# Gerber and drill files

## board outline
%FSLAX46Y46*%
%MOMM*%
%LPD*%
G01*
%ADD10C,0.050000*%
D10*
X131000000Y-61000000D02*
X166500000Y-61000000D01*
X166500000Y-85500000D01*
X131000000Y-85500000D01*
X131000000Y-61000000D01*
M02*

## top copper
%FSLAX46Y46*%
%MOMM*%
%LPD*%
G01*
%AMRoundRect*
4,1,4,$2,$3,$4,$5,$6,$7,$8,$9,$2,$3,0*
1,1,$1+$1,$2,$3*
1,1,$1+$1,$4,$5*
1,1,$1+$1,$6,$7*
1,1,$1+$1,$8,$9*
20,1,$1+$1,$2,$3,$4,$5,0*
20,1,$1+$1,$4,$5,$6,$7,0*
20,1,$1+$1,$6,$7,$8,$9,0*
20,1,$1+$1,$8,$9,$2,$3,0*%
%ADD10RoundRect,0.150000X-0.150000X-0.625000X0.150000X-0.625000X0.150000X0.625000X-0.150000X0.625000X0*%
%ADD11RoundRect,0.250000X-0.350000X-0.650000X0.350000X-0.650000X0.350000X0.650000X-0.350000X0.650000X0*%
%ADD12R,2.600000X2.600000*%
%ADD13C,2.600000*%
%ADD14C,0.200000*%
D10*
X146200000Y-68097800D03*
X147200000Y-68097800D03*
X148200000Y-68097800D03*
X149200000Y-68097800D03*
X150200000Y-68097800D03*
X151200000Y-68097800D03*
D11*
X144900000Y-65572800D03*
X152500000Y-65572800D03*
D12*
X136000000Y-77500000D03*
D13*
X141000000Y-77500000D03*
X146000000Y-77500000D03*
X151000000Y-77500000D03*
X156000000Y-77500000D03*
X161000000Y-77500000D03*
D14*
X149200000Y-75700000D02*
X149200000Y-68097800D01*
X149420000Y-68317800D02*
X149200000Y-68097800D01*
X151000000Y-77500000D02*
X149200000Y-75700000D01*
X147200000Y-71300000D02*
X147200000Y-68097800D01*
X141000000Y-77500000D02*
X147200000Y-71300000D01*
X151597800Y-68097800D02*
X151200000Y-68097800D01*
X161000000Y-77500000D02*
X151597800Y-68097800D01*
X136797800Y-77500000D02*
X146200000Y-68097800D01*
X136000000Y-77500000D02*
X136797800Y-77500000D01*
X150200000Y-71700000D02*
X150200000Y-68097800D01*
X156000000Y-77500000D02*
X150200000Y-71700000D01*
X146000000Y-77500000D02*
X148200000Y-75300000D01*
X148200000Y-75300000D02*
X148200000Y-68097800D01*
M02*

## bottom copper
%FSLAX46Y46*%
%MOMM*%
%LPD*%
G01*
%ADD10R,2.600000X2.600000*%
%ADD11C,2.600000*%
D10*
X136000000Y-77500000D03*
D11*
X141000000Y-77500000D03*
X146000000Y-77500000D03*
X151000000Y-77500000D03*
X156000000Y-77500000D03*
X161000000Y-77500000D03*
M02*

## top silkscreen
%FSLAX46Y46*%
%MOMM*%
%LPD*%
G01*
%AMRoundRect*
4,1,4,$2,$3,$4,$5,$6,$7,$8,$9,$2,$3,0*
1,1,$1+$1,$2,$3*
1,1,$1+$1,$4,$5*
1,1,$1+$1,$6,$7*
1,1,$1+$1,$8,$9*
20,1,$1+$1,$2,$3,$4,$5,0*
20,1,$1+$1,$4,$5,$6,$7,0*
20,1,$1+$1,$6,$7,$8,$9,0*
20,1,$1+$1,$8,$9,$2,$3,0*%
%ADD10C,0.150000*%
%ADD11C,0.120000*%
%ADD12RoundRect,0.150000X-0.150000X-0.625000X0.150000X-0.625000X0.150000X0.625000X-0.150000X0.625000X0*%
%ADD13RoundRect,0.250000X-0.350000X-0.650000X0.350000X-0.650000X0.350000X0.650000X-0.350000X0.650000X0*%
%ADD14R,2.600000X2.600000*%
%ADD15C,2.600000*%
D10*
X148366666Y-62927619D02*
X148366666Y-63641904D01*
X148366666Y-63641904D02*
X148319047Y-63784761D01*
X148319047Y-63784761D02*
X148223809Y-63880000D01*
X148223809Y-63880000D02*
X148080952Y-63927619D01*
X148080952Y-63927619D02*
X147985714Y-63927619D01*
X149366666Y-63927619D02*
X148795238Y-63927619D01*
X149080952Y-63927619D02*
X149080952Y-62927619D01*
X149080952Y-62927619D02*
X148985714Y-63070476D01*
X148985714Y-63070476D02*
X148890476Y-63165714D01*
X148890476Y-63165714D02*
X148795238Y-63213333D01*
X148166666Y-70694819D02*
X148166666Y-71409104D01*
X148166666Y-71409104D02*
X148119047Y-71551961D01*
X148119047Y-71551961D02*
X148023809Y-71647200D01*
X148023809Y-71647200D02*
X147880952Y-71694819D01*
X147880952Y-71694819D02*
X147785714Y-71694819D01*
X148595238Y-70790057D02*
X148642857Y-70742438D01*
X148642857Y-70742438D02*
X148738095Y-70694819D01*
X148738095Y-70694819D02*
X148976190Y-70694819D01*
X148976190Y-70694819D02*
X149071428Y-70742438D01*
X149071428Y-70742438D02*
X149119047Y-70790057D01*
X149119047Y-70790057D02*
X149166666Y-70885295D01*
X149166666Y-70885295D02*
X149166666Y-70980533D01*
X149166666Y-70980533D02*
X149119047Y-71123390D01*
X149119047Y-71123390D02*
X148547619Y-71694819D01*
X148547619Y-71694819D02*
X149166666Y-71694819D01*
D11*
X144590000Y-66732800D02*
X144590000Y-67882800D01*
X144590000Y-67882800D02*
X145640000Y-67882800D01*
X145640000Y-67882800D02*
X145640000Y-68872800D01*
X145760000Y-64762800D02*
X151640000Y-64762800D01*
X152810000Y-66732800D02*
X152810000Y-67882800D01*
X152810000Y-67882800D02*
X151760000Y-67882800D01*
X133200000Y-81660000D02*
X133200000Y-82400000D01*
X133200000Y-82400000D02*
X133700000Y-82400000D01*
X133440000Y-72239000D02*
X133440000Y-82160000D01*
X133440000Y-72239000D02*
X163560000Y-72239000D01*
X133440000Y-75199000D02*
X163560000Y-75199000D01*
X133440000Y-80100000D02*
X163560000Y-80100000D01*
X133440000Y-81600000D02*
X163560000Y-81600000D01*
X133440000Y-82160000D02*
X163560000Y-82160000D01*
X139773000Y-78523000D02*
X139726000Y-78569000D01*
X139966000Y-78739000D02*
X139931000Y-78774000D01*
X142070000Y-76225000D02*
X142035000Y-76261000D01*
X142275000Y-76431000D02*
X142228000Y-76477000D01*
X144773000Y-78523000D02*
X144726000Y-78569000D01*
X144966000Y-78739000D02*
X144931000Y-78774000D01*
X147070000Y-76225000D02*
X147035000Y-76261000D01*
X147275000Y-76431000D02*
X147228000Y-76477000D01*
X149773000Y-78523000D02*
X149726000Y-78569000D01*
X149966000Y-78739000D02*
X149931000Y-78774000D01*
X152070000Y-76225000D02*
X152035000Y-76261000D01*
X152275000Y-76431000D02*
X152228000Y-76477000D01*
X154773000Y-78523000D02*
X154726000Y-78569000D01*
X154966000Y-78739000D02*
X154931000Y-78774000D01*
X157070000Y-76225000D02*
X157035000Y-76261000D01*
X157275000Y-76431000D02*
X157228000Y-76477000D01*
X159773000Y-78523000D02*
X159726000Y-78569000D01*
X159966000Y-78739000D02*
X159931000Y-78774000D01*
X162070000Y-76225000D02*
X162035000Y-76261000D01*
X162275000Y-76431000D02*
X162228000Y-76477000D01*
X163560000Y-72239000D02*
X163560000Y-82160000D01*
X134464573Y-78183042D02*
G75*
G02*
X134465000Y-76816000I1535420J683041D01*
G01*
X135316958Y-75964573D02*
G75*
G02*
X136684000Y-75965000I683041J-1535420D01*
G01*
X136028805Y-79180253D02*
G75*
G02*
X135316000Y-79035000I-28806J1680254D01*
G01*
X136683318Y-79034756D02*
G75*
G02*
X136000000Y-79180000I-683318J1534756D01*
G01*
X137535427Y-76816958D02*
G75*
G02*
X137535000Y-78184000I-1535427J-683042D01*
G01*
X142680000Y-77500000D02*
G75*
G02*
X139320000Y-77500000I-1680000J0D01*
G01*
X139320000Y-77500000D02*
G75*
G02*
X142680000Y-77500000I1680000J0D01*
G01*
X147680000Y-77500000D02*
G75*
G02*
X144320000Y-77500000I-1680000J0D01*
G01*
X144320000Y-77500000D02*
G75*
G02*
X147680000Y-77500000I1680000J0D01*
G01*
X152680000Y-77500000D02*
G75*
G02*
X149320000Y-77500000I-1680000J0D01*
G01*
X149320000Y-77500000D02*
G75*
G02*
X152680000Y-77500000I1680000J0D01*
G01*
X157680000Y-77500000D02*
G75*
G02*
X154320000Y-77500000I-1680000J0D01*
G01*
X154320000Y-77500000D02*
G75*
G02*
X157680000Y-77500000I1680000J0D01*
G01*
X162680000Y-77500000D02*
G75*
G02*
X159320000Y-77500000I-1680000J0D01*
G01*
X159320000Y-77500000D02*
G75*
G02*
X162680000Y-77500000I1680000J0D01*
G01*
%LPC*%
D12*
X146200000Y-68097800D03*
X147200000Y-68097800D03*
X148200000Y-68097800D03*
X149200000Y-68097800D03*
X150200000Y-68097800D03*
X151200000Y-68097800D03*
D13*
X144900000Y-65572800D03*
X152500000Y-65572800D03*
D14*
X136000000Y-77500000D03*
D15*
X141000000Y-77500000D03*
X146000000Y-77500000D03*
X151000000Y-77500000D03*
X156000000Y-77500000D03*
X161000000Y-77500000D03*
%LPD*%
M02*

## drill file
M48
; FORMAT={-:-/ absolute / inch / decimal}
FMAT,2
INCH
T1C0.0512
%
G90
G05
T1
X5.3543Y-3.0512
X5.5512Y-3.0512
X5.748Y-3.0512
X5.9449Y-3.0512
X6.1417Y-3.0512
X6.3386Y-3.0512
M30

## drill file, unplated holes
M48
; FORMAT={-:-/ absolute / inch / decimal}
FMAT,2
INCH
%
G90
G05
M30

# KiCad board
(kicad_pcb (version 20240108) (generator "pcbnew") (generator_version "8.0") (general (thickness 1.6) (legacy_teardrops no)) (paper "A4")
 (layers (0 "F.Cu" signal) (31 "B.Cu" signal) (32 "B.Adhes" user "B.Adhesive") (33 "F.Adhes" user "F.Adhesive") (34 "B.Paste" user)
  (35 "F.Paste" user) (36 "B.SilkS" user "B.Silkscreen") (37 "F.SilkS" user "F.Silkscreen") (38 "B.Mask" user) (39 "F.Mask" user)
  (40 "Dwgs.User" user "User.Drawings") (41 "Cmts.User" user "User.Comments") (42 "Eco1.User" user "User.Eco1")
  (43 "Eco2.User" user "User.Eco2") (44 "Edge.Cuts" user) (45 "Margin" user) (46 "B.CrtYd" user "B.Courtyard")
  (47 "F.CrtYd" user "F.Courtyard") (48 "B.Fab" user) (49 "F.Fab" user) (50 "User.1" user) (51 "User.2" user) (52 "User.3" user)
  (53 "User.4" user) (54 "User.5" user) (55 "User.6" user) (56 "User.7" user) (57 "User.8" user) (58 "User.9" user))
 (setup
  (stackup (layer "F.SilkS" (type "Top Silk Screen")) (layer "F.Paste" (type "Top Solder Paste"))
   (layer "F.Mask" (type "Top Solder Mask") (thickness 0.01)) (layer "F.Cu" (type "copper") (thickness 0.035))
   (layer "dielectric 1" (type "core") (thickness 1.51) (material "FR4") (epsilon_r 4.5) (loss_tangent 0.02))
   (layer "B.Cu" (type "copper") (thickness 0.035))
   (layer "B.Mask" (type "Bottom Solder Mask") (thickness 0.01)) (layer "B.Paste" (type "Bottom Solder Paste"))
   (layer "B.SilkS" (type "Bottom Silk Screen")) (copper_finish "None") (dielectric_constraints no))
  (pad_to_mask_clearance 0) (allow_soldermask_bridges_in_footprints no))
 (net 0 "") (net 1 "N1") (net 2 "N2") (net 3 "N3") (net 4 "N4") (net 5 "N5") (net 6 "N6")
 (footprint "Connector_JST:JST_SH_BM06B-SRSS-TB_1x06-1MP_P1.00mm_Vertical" (layer "F.Cu") (at 148.7 66.7728)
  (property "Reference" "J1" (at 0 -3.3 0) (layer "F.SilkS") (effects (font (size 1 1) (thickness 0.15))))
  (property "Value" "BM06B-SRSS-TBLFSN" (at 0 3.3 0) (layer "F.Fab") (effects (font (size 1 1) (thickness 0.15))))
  (fp_line (start -4.11 -0.04) (end -4.11 1.11) (stroke (width 0.12) (type solid)) (layer "F.SilkS"))
  (fp_line (start -4.11 1.11) (end -3.06 1.11) (stroke (width 0.12) (type solid)) (layer "F.SilkS"))
  (fp_line (start -3.06 1.11) (end -3.06 2.1) (stroke (width 0.12) (type solid)) (layer "F.SilkS"))
  (fp_line (start -2.94 -2.01) (end 2.94 -2.01) (stroke (width 0.12) (type solid)) (layer "F.SilkS"))
  (fp_line (start 4.11 -0.04) (end 4.11 1.11) (stroke (width 0.12) (type solid)) (layer "F.SilkS"))
  (fp_line (start 4.11 1.11) (end 3.06 1.11) (stroke (width 0.12) (type solid)) (layer "F.SilkS"))
  (pad "1" smd roundrect (at -2.5 1.325) (size 0.6 1.55) (layers "F.Cu" "F.Paste" "F.Mask") (roundrect_rratio 0.25) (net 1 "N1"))
  (pad "2" smd roundrect (at -1.5 1.325) (size 0.6 1.55) (layers "F.Cu" "F.Paste" "F.Mask") (roundrect_rratio 0.25) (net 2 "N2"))
  (pad "3" smd roundrect (at -0.5 1.325) (size 0.6 1.55) (layers "F.Cu" "F.Paste" "F.Mask") (roundrect_rratio 0.25) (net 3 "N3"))
  (pad "4" smd roundrect (at 0.5 1.325) (size 0.6 1.55) (layers "F.Cu" "F.Paste" "F.Mask") (roundrect_rratio 0.25) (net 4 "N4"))
  (pad "5" smd roundrect (at 1.5 1.325) (size 0.6 1.55) (layers "F.Cu" "F.Paste" "F.Mask") (roundrect_rratio 0.25) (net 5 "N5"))
  (pad "6" smd roundrect (at 2.5 1.325) (size 0.6 1.55) (layers "F.Cu" "F.Paste" "F.Mask") (roundrect_rratio 0.25) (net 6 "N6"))
  (pad "MP" smd roundrect (at -3.8 -1.2) (size 1.2 1.8) (layers "F.Cu" "F.Paste" "F.Mask") (roundrect_rratio 0.208333))
  (pad "MP" smd roundrect (at 3.8 -1.2) (size 1.2 1.8) (layers "F.Cu" "F.Paste" "F.Mask") (roundrect_rratio 0.208333)))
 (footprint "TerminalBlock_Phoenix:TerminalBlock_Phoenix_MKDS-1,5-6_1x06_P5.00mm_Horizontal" (layer "F.Cu") (at 136 77.5)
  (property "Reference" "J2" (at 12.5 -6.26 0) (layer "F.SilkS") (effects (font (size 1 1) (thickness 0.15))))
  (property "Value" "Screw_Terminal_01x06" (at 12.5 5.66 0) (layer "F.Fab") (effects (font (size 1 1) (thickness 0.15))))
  (fp_line (start -2.8 4.16) (end -2.8 4.9) (stroke (width 0.12) (type solid)) (layer "F.SilkS"))
  (fp_line (start -2.8 4.9) (end -2.3 4.9) (stroke (width 0.12) (type solid)) (layer "F.SilkS"))
  (fp_line (start -2.56 -5.261) (end -2.56 4.66) (stroke (width 0.12) (type solid)) (layer "F.SilkS"))
  (fp_line (start -2.56 -5.261) (end 27.56 -5.261) (stroke (width 0.12) (type solid)) (layer "F.SilkS"))
  (fp_line (start -2.56 -2.301) (end 27.56 -2.301) (stroke (width 0.12) (type solid)) (layer "F.SilkS"))
  (fp_line (start -2.56 2.6) (end 27.56 2.6) (stroke (width 0.12) (type solid)) (layer "F.SilkS"))
  (fp_line (start -2.56 4.1) (end 27.56 4.1) (stroke (width 0.12) (type solid)) (layer "F.SilkS"))
  (fp_line (start -2.56 4.66) (end 27.56 4.66) (stroke (width 0.12) (type solid)) (layer "F.SilkS"))
  (fp_line (start 3.773 1.023) (end 3.726 1.069) (stroke (width 0.12) (type solid)) (layer "F.SilkS"))
  (fp_line (start 3.966 1.239) (end 3.931 1.274) (stroke (width 0.12) (type solid)) (layer "F.SilkS"))
  (fp_line (start 6.07 -1.275) (end 6.035 -1.239) (stroke (width 0.12) (type solid)) (layer "F.SilkS"))
  (fp_line (start 6.275 -1.069) (end 6.228 -1.023) (stroke (width 0.12) (type solid)) (layer "F.SilkS"))
  (fp_line (start 8.773 1.023) (end 8.726 1.069) (stroke (width 0.12) (type solid)) (layer "F.SilkS"))
  (fp_line (start 8.966 1.239) (end 8.931 1.274) (stroke (width 0.12) (type solid)) (layer "F.SilkS"))
  (fp_line (start 11.07 -1.275) (end 11.035 -1.239) (stroke (width 0.12) (type solid)) (layer "F.SilkS"))
  (fp_line (start 11.275 -1.069) (end 11.228 -1.023) (stroke (width 0.12) (type solid)) (layer "F.SilkS"))
  (fp_line (start 13.773 1.023) (end 13.726 1.069) (stroke (width 0.12) (type solid)) (layer "F.SilkS"))
  (fp_line (start 13.966 1.239) (end 13.931 1.274) (stroke (width 0.12) (type solid)) (layer "F.SilkS"))
  (fp_line (start 16.07 -1.275) (end 16.035 -1.239) (stroke (width 0.12) (type solid)) (layer "F.SilkS"))
  (fp_line (start 16.275 -1.069) (end 16.228 -1.023) (stroke (width 0.12) (type solid)) (layer "F.SilkS"))
  (fp_line (start 18.773 1.023) (end 18.726 1.069) (stroke (width 0.12) (type solid)) (layer "F.SilkS"))
  (fp_line (start 18.966 1.239) (end 18.931 1.274) (stroke (width 0.12) (type solid)) (layer "F.SilkS"))
  (fp_line (start 21.07 -1.275) (end 21.035 -1.239) (stroke (width 0.12) (type solid)) (layer "F.SilkS"))
  (fp_line (start 21.275 -1.069) (end 21.228 -1.023) (stroke (width 0.12) (type solid)) (layer "F.SilkS"))
  (fp_line (start 23.773 1.023) (end 23.726 1.069) (stroke (width 0.12) (type solid)) (layer "F.SilkS"))
  (fp_line (start 23.966 1.239) (end 23.931 1.274) (stroke (width 0.12) (type solid)) (layer "F.SilkS"))
  (fp_line (start 26.07 -1.275) (end 26.035 -1.239) (stroke (width 0.12) (type solid)) (layer "F.SilkS"))
  (fp_line (start 26.275 -1.069) (end 26.228 -1.023) (stroke (width 0.12) (type solid)) (layer "F.SilkS"))
  (fp_line (start 27.56 -5.261) (end 27.56 4.66) (stroke (width 0.12) (type solid)) (layer "F.SilkS"))
  (fp_arc (start -1.535427 0.683042) (mid -1.680501 -0.000524) (end -1.535 -0.684) (stroke (width 0.12) (type solid)) (layer "F.SilkS"))
  (fp_arc (start -0.683042 -1.535427) (mid 0.000524 -1.680501) (end 0.684 -1.535) (stroke (width 0.12) (type solid)) (layer "F.SilkS"))
  (fp_arc (start 0.028805 1.680253) (mid -0.335551 1.646659) (end -0.684 1.535) (stroke (width 0.12) (type solid)) (layer "F.SilkS"))
  (fp_arc (start 0.683318 1.534756) (mid 0.349292 1.643288) (end 0 1.68) (stroke (width 0.12) (type solid)) (layer "F.SilkS"))
  (fp_arc (start 1.535427 -0.683042) (mid 1.680501 0.000524) (end 1.535 0.684) (stroke (width 0.12) (type solid)) (layer "F.SilkS"))
  (fp_circle (center 5 0) (end 6.68 0) (stroke (width 0.12) (type solid)) (fill none) (layer "F.SilkS"))
  (fp_circle (center 10 0) (end 11.68 0) (stroke (width 0.12) (type solid)) (fill none) (layer "F.SilkS"))
  (fp_circle (center 15 0) (end 16.68 0) (stroke (width 0.12) (type solid)) (fill none) (layer "F.SilkS"))
  (fp_circle (center 20 0) (end 21.68 0) (stroke (width 0.12) (type solid)) (fill none) (layer "F.SilkS"))
  (fp_circle (center 25 0) (end 26.68 0) (stroke (width 0.12) (type solid)) (fill none) (layer "F.SilkS"))
  (pad "1" thru_hole rect (at 0 0) (size 2.6 2.6) (drill 1.3) (layers "*.Cu" "*.Mask") (remove_unused_layers no) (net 1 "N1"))
  (pad "2" thru_hole circle (at 5 0) (size 2.6 2.6) (drill 1.3) (layers "*.Cu" "*.Mask") (remove_unused_layers no) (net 2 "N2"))
  (pad "3" thru_hole circle (at 10 0) (size 2.6 2.6) (drill 1.3) (layers "*.Cu" "*.Mask") (remove_unused_layers no) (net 3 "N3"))
  (pad "4" thru_hole circle (at 15 0) (size 2.6 2.6) (drill 1.3) (layers "*.Cu" "*.Mask") (remove_unused_layers no) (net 4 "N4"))
  (pad "5" thru_hole circle (at 20 0) (size 2.6 2.6) (drill 1.3) (layers "*.Cu" "*.Mask") (remove_unused_layers no) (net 5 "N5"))
  (pad "6" thru_hole circle (at 25 0) (size 2.6 2.6) (drill 1.3) (layers "*.Cu" "*.Mask") (remove_unused_layers no) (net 6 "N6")))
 (gr_rect (start 131 61) (end 166.5 85.5) (stroke (width 0.05) (type default)) (fill none) (layer "Edge.Cuts"))
 (segment (start 149.2 75.7) (end 149.2 68.0978) (width 0.2) (layer "F.Cu") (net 4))
 (segment (start 149.42 68.3178) (end 149.2 68.0978) (width 0.2) (layer "F.Cu") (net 4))
 (segment (start 151 77.5) (end 149.2 75.7) (width 0.2) (layer "F.Cu") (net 4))
 (segment (start 147.2 71.3) (end 147.2 68.0978) (width 0.2) (layer "F.Cu") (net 2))
 (segment (start 141 77.5) (end 147.2 71.3) (width 0.2) (layer "F.Cu") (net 2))
 (segment (start 151.5978 68.0978) (end 151.2 68.0978) (width 0.2) (layer "F.Cu") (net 6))
 (segment (start 161 77.5) (end 151.5978 68.0978) (width 0.2) (layer "F.Cu") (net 6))
 (segment (start 136.7978 77.5) (end 146.2 68.0978) (width 0.2) (layer "F.Cu") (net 1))
 (segment (start 136 77.5) (end 136.7978 77.5) (width 0.2) (layer "F.Cu") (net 1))
 (segment (start 150.2 71.7) (end 150.2 68.0978) (width 0.2) (layer "F.Cu") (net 5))
 (segment (start 156 77.5) (end 150.2 71.7) (width 0.2) (layer "F.Cu") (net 5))
 (segment (start 146 77.5) (end 148.2 75.3) (width 0.2) (layer "F.Cu") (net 3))
 (segment (start 148.2 75.3) (end 148.2 68.0978) (width 0.2) (layer "F.Cu") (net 3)))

